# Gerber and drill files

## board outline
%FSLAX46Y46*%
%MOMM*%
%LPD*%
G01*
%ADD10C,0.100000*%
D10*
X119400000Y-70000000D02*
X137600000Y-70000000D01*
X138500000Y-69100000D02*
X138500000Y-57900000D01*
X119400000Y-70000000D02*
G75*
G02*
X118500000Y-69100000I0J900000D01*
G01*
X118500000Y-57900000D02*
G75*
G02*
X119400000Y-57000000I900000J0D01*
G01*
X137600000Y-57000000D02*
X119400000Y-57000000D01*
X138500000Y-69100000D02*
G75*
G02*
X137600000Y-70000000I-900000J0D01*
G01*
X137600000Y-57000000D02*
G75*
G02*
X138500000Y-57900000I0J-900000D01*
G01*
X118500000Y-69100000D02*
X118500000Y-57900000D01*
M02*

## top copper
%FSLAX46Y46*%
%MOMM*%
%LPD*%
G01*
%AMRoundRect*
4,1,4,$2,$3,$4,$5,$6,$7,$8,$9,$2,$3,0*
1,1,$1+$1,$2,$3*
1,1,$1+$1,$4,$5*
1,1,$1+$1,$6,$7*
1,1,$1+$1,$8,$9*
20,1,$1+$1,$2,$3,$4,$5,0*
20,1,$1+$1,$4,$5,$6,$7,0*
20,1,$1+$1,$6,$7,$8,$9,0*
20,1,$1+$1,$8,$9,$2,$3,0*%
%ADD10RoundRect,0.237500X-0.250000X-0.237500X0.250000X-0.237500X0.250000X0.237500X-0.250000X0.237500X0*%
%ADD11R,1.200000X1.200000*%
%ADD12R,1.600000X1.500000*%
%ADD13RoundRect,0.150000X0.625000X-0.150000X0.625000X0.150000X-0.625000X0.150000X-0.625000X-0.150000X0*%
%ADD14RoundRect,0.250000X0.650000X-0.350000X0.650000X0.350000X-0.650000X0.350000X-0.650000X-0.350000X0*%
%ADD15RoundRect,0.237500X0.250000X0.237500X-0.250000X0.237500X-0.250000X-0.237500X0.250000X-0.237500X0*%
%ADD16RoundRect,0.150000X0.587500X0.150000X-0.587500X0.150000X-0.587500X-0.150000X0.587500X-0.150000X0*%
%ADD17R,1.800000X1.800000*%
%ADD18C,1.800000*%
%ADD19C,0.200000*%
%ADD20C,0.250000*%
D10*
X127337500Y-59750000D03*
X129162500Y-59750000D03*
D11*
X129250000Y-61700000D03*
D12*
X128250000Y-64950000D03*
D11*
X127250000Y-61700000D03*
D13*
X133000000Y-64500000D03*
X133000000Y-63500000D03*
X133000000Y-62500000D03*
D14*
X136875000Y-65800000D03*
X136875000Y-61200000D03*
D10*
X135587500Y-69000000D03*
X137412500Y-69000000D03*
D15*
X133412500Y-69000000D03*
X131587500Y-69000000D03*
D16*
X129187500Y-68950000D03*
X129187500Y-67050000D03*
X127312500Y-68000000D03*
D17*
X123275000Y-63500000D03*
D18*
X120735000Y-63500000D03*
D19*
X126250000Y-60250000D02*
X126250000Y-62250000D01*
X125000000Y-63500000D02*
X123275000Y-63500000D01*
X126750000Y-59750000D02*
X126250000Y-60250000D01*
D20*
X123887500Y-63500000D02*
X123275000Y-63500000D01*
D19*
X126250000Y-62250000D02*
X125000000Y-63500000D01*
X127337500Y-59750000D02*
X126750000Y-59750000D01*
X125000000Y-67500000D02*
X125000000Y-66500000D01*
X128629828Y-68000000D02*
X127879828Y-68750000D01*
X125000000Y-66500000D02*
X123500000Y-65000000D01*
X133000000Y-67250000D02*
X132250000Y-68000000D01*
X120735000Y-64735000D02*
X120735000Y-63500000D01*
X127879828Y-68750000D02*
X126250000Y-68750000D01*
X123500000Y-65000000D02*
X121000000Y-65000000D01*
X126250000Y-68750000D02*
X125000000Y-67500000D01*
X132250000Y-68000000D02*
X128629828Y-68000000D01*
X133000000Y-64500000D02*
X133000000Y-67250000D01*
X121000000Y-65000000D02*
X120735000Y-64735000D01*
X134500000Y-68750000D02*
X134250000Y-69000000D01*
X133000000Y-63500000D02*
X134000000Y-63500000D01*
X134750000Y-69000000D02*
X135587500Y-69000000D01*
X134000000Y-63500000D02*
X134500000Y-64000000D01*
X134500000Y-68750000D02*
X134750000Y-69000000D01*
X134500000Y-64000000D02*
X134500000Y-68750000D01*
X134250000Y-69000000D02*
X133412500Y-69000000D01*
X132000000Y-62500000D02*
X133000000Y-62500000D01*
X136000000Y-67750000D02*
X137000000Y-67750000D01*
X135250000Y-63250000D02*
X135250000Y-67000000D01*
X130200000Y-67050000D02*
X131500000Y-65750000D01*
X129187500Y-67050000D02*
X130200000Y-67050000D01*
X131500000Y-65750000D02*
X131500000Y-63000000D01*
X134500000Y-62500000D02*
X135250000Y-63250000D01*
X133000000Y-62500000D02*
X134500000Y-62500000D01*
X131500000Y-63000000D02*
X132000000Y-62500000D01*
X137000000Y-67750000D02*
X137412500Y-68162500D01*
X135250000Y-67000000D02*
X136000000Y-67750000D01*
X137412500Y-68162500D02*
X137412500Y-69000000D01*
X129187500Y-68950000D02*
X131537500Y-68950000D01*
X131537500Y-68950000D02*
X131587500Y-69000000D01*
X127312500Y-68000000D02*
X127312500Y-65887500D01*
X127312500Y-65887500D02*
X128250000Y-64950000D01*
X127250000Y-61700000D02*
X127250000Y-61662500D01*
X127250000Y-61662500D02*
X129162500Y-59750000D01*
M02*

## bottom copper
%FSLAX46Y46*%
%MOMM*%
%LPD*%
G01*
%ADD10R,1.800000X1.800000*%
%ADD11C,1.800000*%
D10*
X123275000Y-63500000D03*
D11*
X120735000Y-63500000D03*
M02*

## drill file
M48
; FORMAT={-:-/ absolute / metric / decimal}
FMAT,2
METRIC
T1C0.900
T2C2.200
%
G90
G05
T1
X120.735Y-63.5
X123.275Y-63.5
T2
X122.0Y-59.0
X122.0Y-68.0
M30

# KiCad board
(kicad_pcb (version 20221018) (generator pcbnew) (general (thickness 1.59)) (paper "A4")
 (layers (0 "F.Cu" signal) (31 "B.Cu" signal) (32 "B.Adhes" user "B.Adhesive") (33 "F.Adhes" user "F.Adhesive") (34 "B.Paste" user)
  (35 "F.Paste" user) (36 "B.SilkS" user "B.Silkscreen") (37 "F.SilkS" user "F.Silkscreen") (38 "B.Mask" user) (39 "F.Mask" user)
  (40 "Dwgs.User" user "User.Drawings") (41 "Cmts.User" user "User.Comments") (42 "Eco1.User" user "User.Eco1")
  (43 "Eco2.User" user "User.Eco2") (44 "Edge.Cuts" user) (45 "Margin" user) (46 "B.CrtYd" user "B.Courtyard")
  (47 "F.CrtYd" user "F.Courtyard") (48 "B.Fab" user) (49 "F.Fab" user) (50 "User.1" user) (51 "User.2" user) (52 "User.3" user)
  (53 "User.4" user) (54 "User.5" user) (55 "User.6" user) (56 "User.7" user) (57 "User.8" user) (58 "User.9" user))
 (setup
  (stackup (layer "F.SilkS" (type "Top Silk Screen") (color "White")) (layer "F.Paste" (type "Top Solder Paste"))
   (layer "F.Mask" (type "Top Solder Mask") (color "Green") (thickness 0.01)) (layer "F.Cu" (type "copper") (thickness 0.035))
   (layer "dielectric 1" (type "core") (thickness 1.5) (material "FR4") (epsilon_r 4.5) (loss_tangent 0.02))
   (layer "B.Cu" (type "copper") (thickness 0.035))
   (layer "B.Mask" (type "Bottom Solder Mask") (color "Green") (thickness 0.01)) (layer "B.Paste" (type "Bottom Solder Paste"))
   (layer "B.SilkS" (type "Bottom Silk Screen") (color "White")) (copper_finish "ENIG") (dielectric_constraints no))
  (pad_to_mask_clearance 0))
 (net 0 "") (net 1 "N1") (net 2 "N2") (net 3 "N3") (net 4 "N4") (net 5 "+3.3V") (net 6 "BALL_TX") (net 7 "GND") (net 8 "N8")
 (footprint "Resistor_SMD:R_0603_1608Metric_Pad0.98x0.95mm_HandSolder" (layer "F.Cu") (at 128.25 59.75)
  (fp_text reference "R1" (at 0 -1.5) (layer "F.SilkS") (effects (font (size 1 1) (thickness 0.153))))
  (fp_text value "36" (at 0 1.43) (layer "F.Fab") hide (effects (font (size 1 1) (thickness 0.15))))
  (pad "1" smd roundrect (at -0.9125 0) (size 0.975 0.95) (layers "F.Cu" "F.Paste" "F.Mask") (roundrect_rratio 0.25) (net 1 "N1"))
  (pad "2" smd roundrect (at 0.9125 0) (size 0.975 0.95) (layers "F.Cu" "F.Paste" "F.Mask") (roundrect_rratio 0.25) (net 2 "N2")))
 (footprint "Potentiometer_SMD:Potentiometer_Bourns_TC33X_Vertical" (layer "F.Cu") (at 128.25 63.5 -90)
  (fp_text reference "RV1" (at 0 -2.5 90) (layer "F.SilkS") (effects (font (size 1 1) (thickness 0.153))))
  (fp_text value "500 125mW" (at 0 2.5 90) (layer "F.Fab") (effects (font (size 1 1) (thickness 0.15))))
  (pad "1" smd rect (at -1.8 -1 270) (size 1.2 1.2) (layers "F.Cu" "F.Paste" "F.Mask") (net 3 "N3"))
  (pad "2" smd rect (at 1.45 0 270) (size 1.5 1.6) (layers "F.Cu" "F.Paste" "F.Mask") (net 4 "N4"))
  (pad "3" smd rect (at -1.8 1 270) (size 1.2 1.2) (layers "F.Cu" "F.Paste" "F.Mask") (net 2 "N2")))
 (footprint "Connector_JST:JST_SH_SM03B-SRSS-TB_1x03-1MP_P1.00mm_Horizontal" (layer "F.Cu") (at 135 63.5 90)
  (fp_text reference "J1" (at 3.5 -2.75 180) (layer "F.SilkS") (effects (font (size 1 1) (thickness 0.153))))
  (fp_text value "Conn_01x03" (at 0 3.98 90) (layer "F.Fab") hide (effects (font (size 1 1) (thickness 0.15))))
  (pad "1" smd roundrect (at -1 -2 90) (size 0.6 1.55) (layers "F.Cu" "F.Paste" "F.Mask") (roundrect_rratio 0.25) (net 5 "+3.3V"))
  (pad "2" smd roundrect (at 0 -2 90) (size 0.6 1.55) (layers "F.Cu" "F.Paste" "F.Mask") (roundrect_rratio 0.25) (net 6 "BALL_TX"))
  (pad "3" smd roundrect (at 1 -2 90) (size 0.6 1.55) (layers "F.Cu" "F.Paste" "F.Mask") (roundrect_rratio 0.25) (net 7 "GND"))
  (pad "MP" smd roundrect (at -2.3 1.875 90) (size 1.2 1.8) (layers "F.Cu" "F.Paste" "F.Mask") (roundrect_rratio 0.2083333333))
  (pad "MP" smd roundrect (at 2.3 1.875 90) (size 1.2 1.8) (layers "F.Cu" "F.Paste" "F.Mask") (roundrect_rratio 0.2083333333)))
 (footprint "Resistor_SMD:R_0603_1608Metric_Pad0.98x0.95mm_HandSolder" (layer "F.Cu") (at 136.5 69)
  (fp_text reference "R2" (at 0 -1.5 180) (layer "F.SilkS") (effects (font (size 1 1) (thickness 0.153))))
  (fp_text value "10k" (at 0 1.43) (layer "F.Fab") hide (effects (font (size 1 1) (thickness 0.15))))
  (pad "1" smd roundrect (at -0.9125 0) (size 0.975 0.95) (layers "F.Cu" "F.Paste" "F.Mask") (roundrect_rratio 0.25) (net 6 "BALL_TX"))
  (pad "2" smd roundrect (at 0.9125 0) (size 0.975 0.95) (layers "F.Cu" "F.Paste" "F.Mask") (roundrect_rratio 0.25) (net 7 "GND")))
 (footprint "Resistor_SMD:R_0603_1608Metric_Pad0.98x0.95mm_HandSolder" (layer "F.Cu") (at 132.5 69 180)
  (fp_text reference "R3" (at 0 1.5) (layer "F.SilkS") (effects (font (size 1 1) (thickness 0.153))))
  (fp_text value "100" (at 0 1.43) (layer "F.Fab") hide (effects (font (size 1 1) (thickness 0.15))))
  (pad "1" smd roundrect (at -0.9125 0 180) (size 0.975 0.95) (layers "F.Cu" "F.Paste" "F.Mask") (roundrect_rratio 0.25) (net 6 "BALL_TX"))
  (pad "2" smd roundrect (at 0.9125 0 180) (size 0.975 0.95) (layers "F.Cu" "F.Paste" "F.Mask") (roundrect_rratio 0.25) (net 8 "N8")))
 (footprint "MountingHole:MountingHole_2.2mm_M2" (layer "F.Cu") (at 122 68 -90)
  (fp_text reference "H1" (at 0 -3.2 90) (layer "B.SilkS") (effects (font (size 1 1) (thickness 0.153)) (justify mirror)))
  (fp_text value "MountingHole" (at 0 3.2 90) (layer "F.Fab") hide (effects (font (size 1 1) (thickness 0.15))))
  (pad "" np_thru_hole circle (at 0 0 270) (size 2.2 2.2) (drill 2.2) (layers "*.Cu" "*.Mask")))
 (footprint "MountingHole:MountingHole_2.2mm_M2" (layer "F.Cu") (at 122 59 -90)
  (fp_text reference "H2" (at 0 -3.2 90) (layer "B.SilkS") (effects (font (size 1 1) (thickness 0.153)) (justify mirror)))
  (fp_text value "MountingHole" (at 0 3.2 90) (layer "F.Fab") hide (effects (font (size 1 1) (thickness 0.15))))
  (pad "" np_thru_hole circle (at 0 0 270) (size 2.2 2.2) (drill 2.2) (layers "*.Cu" "*.Mask")))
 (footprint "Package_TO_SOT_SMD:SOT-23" (layer "F.Cu") (at 128.25 68 180)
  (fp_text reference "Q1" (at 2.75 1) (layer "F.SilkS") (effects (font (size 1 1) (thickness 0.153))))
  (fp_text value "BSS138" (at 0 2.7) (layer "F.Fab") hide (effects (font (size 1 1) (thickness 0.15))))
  (pad "1" smd roundrect (at -0.9375 -0.95 180) (size 1.475 0.6) (layers "F.Cu" "F.Paste" "F.Mask") (roundrect_rratio 0.25) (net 8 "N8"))
  (pad "2" smd roundrect (at -0.9375 0.95 180) (size 1.475 0.6) (layers "F.Cu" "F.Paste" "F.Mask") (roundrect_rratio 0.25) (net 7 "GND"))
  (pad "3" smd roundrect (at 0.9375 0 180) (size 1.475 0.6) (layers "F.Cu" "F.Paste" "F.Mask") (roundrect_rratio 0.25) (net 4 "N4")))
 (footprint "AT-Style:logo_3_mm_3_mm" (layer "B.Cu") (at 135.5 60.5 180)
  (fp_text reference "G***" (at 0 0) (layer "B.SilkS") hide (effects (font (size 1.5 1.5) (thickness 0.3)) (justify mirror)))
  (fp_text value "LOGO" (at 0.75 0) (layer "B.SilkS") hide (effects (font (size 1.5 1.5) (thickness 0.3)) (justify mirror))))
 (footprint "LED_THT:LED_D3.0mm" (layer "B.Cu") (at 123.275 63.5 180)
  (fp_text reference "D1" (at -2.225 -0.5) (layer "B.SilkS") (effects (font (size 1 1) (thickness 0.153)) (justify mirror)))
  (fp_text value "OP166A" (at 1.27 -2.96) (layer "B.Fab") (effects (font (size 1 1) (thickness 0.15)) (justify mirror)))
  (pad "1" thru_hole rect (at 0 0 180) (size 1.8 1.8) (drill 0.9) (layers "*.Cu" "*.Mask") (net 1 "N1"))
  (pad "2" thru_hole circle (at 2.54 0 180) (size 1.8 1.8) (drill 0.9) (layers "*.Cu" "*.Mask") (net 5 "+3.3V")))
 (gr_line (start 119.4 70) (end 137.6 70) (stroke (width 0.1) (type default)) (layer "Edge.Cuts"))
 (gr_line (start 138.5 69.1) (end 138.5 57.9) (stroke (width 0.1) (type default)) (layer "Edge.Cuts"))
 (gr_arc (start 119.4 70) (mid 118.763604 69.736396) (end 118.5 69.1) (stroke (width 0.1) (type default)) (layer "Edge.Cuts"))
 (gr_arc (start 118.5 57.9) (mid 118.763604 57.263604) (end 119.4 57) (stroke (width 0.1) (type default)) (layer "Edge.Cuts"))
 (gr_line (start 137.6 57) (end 119.4 57) (stroke (width 0.1) (type default)) (layer "Edge.Cuts"))
 (gr_arc (start 138.5 69.1) (mid 138.236396 69.736396) (end 137.6 70) (stroke (width 0.1) (type default)) (layer "Edge.Cuts"))
 (gr_arc (start 137.6 57) (mid 138.236396 57.263604) (end 138.5 57.9) (stroke (width 0.1) (type default)) (layer "Edge.Cuts"))
 (gr_line (start 118.5 69.1) (end 118.5 57.9) (stroke (width 0.1) (type default)) (layer "Edge.Cuts"))
 (segment (start 126.25 60.25) (end 126.25 62.25) (width 0.2) (layer "F.Cu") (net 1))
 (segment (start 125 63.5) (end 123.275 63.5) (width 0.2) (layer "F.Cu") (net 1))
 (segment (start 126.75 59.75) (end 126.25 60.25) (width 0.2) (layer "F.Cu") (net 1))
 (segment (start 123.8875 63.5) (end 123.275 63.5) (width 0.25) (layer "F.Cu") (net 1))
 (segment (start 126.25 62.25) (end 125 63.5) (width 0.2) (layer "F.Cu") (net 1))
 (segment (start 127.3375 59.75) (end 126.75 59.75) (width 0.2) (layer "F.Cu") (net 1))
 (segment (start 125 67.5) (end 125 66.5) (width 0.2) (layer "F.Cu") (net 5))
 (segment (start 128.629828 68) (end 127.879828 68.75) (width 0.2) (layer "F.Cu") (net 5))
 (segment (start 125 66.5) (end 123.5 65) (width 0.2) (layer "F.Cu") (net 5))
 (segment (start 133 67.25) (end 132.25 68) (width 0.2) (layer "F.Cu") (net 5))
 (segment (start 120.735 64.735) (end 120.735 63.5) (width 0.2) (layer "F.Cu") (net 5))
 (segment (start 127.879828 68.75) (end 126.25 68.75) (width 0.2) (layer "F.Cu") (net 5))
 (segment (start 123.5 65) (end 121 65) (width 0.2) (layer "F.Cu") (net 5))
 (segment (start 126.25 68.75) (end 125 67.5) (width 0.2) (layer "F.Cu") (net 5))
 (segment (start 132.25 68) (end 128.629828 68) (width 0.2) (layer "F.Cu") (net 5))
 (segment (start 133 64.5) (end 133 67.25) (width 0.2) (layer "F.Cu") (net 5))
 (segment (start 121 65) (end 120.735 64.735) (width 0.2) (layer "F.Cu") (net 5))
 (segment (start 134.5 68.75) (end 134.25 69) (width 0.2) (layer "F.Cu") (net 6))
 (segment (start 133 63.5) (end 134 63.5) (width 0.2) (layer "F.Cu") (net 6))
 (segment (start 134.75 69) (end 135.5875 69) (width 0.2) (layer "F.Cu") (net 6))
 (segment (start 134 63.5) (end 134.5 64) (width 0.2) (layer "F.Cu") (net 6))
 (segment (start 134.5 68.75) (end 134.75 69) (width 0.2) (layer "F.Cu") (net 6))
 (segment (start 134.5 64) (end 134.5 68.75) (width 0.2) (layer "F.Cu") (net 6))
 (segment (start 134.25 69) (end 133.4125 69) (width 0.2) (layer "F.Cu") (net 6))
 (segment (start 132 62.5) (end 133 62.5) (width 0.2) (layer "F.Cu") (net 7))
 (segment (start 136 67.75) (end 137 67.75) (width 0.2) (layer "F.Cu") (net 7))
 (segment (start 135.25 63.25) (end 135.25 67) (width 0.2) (layer "F.Cu") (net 7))
 (segment (start 130.2 67.05) (end 131.5 65.75) (width 0.2) (layer "F.Cu") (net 7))
 (segment (start 129.1875 67.05) (end 130.2 67.05) (width 0.2) (layer "F.Cu") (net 7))
 (segment (start 131.5 65.75) (end 131.5 63) (width 0.2) (layer "F.Cu") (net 7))
 (segment (start 134.5 62.5) (end 135.25 63.25) (width 0.2) (layer "F.Cu") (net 7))
 (segment (start 133 62.5) (end 134.5 62.5) (width 0.2) (layer "F.Cu") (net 7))
 (segment (start 131.5 63) (end 132 62.5) (width 0.2) (layer "F.Cu") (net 7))
 (segment (start 137 67.75) (end 137.4125 68.1625) (width 0.2) (layer "F.Cu") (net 7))
 (segment (start 135.25 67) (end 136 67.75) (width 0.2) (layer "F.Cu") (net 7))
 (segment (start 137.4125 68.1625) (end 137.4125 69) (width 0.2) (layer "F.Cu") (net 7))
 (segment (start 129.1875 68.95) (end 131.5375 68.95) (width 0.2) (layer "F.Cu") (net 8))
 (segment (start 131.5375 68.95) (end 131.5875 69) (width 0.2) (layer "F.Cu") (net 8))
 (segment (start 127.3125 68) (end 127.3125 65.8875) (width 0.2) (layer "F.Cu") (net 4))
 (segment (start 127.3125 65.8875) (end 128.25 64.95) (width 0.2) (layer "F.Cu") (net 4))
 (segment (start 127.25 61.7) (end 127.25 61.6625) (width 0.2) (layer "F.Cu") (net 2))
 (segment (start 127.25 61.6625) (end 129.1625 59.75) (width 0.2) (layer "F.Cu") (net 2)))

